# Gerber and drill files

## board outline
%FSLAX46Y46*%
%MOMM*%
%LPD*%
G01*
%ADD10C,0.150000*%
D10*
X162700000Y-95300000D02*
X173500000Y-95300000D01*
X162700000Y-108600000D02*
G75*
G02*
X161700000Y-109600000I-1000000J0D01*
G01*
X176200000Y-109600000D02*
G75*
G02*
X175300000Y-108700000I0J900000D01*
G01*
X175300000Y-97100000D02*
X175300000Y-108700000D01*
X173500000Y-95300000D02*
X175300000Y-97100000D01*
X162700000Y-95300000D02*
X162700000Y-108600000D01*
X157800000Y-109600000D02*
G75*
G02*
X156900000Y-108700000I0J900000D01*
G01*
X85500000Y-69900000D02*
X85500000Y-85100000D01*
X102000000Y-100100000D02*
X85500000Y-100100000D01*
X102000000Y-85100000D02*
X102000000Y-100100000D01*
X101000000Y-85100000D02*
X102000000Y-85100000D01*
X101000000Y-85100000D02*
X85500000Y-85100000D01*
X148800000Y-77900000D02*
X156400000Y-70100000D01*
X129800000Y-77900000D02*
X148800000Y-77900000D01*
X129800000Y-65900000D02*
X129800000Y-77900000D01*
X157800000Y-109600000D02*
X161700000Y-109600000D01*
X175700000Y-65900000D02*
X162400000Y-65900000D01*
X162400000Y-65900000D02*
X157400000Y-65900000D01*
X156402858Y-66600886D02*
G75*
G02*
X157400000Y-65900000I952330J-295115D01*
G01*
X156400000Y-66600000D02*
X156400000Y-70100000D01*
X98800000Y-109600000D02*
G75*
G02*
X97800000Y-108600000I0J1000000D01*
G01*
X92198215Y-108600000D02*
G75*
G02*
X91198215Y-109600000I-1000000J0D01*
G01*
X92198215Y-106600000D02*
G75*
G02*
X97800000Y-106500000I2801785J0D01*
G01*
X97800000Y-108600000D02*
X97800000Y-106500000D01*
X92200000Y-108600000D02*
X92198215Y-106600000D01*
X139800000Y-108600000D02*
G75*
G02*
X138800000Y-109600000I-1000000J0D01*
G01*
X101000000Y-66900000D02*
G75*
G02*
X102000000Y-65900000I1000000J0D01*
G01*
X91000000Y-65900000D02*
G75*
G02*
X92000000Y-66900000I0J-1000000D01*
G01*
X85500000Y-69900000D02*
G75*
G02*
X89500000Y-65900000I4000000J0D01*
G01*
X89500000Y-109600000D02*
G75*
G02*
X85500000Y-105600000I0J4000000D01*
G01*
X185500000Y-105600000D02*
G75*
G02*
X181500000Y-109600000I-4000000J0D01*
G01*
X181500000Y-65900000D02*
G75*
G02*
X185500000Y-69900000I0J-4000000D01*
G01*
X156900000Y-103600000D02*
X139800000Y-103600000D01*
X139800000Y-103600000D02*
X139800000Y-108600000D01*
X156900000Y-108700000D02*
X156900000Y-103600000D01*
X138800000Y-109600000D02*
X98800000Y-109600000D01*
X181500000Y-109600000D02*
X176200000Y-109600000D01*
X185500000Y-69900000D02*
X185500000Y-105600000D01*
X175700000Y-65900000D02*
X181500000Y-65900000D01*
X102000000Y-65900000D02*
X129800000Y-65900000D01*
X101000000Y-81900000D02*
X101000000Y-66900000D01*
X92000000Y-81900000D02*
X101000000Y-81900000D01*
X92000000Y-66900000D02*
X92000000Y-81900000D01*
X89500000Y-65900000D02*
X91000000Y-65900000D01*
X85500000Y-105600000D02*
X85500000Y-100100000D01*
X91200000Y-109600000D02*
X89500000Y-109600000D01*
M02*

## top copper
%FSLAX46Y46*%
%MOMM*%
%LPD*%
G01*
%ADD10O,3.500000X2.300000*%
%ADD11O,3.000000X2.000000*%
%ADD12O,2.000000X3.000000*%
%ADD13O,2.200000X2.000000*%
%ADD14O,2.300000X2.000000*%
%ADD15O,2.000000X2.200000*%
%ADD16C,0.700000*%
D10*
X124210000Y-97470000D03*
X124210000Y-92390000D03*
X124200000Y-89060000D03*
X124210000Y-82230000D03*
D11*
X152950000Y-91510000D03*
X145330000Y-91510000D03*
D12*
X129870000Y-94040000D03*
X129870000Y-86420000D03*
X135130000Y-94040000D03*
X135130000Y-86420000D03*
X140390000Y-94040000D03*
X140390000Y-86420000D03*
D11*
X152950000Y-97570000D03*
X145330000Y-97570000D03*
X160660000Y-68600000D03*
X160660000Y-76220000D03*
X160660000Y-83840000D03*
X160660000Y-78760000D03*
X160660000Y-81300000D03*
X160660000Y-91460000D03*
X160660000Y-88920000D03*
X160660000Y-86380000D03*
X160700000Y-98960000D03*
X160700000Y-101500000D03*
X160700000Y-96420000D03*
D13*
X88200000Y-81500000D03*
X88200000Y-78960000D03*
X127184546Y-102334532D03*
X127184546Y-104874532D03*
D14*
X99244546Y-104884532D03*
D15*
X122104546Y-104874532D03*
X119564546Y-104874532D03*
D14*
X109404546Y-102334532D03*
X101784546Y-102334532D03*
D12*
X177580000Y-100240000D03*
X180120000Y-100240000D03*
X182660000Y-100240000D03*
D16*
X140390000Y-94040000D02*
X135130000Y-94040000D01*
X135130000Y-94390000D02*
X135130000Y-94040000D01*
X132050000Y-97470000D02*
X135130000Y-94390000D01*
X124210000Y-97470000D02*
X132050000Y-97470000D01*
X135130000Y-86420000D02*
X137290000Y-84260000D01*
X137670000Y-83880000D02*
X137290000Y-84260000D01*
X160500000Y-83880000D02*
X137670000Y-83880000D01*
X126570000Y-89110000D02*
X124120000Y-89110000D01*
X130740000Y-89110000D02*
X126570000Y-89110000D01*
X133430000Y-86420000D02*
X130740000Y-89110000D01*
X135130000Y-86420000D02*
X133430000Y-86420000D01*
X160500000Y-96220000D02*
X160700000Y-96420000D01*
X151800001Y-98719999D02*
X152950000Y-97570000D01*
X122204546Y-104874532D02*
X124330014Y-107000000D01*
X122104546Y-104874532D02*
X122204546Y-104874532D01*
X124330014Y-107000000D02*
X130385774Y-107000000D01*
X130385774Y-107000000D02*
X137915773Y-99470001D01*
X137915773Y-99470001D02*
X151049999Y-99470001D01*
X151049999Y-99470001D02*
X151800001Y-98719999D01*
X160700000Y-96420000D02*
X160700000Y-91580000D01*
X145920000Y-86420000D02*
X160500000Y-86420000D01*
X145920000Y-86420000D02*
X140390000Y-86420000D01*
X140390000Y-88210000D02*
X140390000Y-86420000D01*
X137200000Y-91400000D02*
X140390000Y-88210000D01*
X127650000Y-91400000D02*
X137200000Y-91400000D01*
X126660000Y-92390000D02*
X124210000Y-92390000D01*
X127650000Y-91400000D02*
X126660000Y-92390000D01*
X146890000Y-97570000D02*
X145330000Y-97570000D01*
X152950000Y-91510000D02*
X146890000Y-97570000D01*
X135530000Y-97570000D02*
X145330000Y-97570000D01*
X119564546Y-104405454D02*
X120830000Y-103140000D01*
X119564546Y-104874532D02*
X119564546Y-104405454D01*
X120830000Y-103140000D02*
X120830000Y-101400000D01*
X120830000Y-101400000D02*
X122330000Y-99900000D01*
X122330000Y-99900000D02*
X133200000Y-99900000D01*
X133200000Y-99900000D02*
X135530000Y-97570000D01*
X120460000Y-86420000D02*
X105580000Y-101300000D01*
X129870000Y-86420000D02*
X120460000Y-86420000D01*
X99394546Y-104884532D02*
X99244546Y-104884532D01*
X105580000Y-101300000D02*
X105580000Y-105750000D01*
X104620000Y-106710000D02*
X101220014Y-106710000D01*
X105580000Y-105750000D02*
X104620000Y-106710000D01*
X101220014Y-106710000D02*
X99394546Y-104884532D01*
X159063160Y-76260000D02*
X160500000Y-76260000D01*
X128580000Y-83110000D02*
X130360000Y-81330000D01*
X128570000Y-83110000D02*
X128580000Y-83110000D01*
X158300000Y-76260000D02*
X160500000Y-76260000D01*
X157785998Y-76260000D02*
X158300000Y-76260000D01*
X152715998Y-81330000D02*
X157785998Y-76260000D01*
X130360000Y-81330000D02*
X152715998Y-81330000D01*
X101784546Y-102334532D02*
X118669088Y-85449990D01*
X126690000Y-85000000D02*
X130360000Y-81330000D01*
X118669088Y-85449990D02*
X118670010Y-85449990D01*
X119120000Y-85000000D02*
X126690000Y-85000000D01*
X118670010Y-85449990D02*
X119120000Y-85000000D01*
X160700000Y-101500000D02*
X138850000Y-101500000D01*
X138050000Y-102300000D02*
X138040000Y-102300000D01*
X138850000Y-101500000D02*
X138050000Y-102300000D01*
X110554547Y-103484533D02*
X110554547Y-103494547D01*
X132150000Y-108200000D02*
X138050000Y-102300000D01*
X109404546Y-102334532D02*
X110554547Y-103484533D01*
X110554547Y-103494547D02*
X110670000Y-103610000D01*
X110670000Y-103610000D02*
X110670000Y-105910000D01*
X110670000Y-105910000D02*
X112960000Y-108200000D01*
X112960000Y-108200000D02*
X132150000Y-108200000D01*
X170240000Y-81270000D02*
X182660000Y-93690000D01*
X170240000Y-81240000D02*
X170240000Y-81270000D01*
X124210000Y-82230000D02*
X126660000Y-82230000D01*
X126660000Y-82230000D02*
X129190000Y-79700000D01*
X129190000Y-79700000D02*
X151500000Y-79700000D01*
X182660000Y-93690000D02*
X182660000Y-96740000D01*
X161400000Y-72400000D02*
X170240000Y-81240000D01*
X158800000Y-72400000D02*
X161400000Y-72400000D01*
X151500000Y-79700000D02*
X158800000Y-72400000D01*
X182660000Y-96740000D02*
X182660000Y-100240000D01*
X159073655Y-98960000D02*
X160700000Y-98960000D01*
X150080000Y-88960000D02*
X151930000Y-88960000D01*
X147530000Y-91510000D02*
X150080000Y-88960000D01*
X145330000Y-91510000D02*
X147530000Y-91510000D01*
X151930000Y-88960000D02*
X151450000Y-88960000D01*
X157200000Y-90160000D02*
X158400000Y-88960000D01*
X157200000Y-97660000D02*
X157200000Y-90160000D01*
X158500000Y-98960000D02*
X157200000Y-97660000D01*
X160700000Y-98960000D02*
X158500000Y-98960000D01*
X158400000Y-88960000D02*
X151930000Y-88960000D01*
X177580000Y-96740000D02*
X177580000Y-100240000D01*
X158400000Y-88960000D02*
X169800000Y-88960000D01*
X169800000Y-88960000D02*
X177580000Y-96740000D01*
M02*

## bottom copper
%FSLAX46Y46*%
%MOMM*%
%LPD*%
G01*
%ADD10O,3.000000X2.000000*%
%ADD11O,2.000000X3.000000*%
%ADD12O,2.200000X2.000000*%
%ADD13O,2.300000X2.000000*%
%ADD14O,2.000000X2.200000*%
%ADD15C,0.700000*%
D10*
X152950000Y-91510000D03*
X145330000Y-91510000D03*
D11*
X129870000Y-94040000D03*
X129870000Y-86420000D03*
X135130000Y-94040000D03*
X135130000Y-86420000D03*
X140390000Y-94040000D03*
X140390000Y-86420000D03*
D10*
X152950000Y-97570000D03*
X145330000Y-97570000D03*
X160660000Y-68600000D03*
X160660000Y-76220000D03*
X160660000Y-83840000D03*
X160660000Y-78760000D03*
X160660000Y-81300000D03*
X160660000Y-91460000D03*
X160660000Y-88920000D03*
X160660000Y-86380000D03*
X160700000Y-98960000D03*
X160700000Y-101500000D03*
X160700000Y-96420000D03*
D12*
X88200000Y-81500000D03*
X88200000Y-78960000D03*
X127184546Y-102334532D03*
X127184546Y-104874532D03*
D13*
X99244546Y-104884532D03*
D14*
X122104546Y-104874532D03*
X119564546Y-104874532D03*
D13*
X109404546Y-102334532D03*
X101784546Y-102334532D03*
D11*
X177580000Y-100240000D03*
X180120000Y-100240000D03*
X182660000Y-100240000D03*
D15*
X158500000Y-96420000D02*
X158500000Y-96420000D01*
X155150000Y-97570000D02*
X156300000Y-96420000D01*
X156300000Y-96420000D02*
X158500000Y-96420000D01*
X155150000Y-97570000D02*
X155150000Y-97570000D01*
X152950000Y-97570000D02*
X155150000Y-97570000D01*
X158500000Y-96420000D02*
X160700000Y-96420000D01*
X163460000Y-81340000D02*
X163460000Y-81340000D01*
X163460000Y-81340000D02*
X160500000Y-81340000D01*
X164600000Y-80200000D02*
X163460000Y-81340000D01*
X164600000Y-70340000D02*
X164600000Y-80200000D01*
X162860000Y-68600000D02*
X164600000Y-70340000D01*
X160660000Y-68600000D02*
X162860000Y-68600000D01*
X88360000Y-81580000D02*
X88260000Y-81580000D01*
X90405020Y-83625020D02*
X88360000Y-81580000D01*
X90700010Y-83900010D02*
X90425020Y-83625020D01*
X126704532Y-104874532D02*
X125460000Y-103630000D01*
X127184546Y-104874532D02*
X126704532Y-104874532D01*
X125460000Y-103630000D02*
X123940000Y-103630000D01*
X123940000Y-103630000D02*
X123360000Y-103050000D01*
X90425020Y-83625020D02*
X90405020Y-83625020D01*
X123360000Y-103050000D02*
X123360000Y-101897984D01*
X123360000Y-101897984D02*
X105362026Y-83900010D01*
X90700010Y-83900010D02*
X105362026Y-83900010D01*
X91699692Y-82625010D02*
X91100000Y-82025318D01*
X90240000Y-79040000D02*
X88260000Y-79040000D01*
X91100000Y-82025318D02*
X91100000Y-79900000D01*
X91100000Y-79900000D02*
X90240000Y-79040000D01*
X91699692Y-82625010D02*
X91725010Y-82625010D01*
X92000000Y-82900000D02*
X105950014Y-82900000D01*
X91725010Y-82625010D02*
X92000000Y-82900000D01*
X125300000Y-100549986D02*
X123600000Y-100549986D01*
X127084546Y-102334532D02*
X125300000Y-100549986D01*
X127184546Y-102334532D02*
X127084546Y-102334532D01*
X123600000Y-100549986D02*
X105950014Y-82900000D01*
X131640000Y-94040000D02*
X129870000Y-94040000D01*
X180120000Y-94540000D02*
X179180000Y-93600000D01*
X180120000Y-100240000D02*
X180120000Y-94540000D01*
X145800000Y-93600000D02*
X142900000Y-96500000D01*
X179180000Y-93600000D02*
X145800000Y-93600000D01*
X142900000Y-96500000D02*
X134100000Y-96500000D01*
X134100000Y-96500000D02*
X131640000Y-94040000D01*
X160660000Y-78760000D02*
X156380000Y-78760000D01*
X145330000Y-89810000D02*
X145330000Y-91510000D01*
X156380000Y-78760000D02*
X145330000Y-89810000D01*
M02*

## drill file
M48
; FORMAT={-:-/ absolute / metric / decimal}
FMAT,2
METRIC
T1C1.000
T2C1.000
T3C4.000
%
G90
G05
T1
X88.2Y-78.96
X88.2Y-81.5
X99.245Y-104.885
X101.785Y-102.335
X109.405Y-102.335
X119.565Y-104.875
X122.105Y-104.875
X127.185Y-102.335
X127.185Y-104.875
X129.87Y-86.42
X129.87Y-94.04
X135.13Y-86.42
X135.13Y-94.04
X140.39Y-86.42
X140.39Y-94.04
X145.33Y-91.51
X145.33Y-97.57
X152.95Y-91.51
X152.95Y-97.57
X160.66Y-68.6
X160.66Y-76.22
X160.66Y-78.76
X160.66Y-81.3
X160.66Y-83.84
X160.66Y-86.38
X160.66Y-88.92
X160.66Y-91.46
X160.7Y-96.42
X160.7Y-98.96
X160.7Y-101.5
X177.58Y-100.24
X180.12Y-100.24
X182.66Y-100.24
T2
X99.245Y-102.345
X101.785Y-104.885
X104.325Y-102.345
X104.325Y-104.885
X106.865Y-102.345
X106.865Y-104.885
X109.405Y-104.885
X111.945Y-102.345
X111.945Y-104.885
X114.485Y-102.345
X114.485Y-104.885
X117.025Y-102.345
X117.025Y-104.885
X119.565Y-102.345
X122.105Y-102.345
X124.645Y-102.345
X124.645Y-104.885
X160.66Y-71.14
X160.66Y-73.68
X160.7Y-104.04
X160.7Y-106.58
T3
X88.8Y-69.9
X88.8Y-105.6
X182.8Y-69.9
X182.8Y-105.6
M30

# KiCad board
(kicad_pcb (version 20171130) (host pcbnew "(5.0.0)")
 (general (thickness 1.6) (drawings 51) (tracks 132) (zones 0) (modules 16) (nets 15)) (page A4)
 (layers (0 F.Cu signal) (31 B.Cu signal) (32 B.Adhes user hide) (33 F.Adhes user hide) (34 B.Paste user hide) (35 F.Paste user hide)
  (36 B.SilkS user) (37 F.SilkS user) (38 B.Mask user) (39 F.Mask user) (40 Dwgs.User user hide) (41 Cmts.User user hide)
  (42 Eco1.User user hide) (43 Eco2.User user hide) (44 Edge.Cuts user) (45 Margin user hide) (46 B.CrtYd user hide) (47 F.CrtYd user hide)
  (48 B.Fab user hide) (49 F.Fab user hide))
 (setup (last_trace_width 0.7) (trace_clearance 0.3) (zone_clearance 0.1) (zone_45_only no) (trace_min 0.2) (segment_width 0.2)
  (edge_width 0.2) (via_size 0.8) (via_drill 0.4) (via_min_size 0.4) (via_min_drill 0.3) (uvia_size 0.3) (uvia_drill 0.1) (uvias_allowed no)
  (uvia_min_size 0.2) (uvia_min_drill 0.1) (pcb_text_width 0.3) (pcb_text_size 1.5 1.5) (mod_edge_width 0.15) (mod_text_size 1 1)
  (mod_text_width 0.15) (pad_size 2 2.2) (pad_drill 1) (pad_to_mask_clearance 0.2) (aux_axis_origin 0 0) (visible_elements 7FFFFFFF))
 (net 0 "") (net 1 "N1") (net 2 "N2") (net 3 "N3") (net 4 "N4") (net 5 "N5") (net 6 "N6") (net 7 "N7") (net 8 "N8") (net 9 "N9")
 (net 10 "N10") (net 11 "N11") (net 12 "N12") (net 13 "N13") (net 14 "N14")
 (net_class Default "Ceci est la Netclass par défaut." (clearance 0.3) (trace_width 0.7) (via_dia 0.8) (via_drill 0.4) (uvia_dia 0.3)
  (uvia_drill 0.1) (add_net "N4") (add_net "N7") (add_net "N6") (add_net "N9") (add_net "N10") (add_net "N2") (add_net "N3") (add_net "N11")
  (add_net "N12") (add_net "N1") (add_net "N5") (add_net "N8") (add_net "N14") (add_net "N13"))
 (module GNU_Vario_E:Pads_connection (layer F.Cu) (at 124.21 84.77)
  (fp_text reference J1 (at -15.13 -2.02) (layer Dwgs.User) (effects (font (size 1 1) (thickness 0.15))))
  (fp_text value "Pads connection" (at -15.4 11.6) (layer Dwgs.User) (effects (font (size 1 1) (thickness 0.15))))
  (pad 5 smd oval (at 0 12.7) (size 3.5 2.3) (layers F.Cu F.Mask) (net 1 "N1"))
  (pad 4 smd oval (at 0 7.62) (size 3.5 2.3) (layers F.Cu F.Mask) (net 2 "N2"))
  (pad 3 smd oval (at -0.01 4.29) (size 3.5 2.3) (layers F.Cu F.Mask) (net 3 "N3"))
  (pad 1 smd oval (at 0 -2.54) (size 3.5 2.3) (layers F.Cu F.Mask) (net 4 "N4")))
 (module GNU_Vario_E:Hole (layer F.Cu) (at 182.8 105.6)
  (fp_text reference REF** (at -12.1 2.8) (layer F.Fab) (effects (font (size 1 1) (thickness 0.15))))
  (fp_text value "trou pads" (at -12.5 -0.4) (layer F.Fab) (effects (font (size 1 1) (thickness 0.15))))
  (pad "" np_thru_hole circle (at 0 0) (size 4 4) (drill 4) (layers *.Cu *.Mask)))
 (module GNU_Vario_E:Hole (layer F.Cu) (at 182.8 69.9)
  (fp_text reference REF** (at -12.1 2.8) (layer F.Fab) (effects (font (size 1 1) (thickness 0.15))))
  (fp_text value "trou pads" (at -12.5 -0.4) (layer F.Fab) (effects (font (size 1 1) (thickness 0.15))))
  (pad "" np_thru_hole circle (at 0 0) (size 4 4) (drill 4) (layers *.Cu *.Mask)))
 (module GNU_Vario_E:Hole (layer F.Cu) (at 88.8 69.9)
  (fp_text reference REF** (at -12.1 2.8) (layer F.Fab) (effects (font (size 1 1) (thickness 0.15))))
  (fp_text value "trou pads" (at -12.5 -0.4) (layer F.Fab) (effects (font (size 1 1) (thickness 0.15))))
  (pad "" np_thru_hole circle (at 0 0) (size 4 4) (drill 4) (layers *.Cu *.Mask)))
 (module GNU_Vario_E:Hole (layer F.Cu) (at 88.8 105.6)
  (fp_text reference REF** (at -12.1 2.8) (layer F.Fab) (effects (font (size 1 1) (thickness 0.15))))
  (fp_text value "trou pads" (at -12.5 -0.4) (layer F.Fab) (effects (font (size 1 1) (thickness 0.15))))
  (pad "" np_thru_hole circle (at 0 0) (size 4 4) (drill 4) (layers *.Cu *.Mask)))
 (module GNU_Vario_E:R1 (layer F.Cu) (at 145.33 91.51 270)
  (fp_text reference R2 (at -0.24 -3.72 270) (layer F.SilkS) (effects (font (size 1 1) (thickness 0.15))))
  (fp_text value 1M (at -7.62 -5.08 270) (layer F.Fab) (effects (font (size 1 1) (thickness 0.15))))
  (pad 2 thru_hole oval (at 0 -7.62 270) (size 2 3) (drill 1) (layers *.Cu *.Mask) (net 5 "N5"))
  (pad 1 thru_hole oval (at 0 0 270) (size 2 3) (drill 1) (layers *.Cu *.Mask) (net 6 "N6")))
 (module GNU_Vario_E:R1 (layer F.Cu) (at 129.87 86.42 180)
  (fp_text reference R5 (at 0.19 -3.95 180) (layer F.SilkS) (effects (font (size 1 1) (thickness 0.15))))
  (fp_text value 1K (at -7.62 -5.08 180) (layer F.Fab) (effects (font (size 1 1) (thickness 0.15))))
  (pad 2 thru_hole oval (at 0 -7.62 180) (size 2 3) (drill 1) (layers *.Cu *.Mask) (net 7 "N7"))
  (pad 1 thru_hole oval (at 0 0 180) (size 2 3) (drill 1) (layers *.Cu *.Mask) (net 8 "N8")))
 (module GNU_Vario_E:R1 (layer F.Cu) (at 135.13 86.42 180)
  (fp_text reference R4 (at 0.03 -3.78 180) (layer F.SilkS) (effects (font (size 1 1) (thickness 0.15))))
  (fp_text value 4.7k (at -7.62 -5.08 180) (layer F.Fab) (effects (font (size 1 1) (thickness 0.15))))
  (pad 2 thru_hole oval (at 0 -7.62 180) (size 2 3) (drill 1) (layers *.Cu *.Mask) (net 1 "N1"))
  (pad 1 thru_hole oval (at 0 0 180) (size 2 3) (drill 1) (layers *.Cu *.Mask) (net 3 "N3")))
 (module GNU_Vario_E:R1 (layer F.Cu) (at 140.39 86.42 180)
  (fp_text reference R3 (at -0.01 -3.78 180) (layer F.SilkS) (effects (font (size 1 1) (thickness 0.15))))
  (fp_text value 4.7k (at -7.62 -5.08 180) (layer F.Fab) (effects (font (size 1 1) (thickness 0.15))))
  (pad 2 thru_hole oval (at 0 -7.62 180) (size 2 3) (drill 1) (layers *.Cu *.Mask) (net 1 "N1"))
  (pad 1 thru_hole oval (at 0 0 180) (size 2 3) (drill 1) (layers *.Cu *.Mask) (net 2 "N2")))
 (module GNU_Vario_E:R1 (layer F.Cu) (at 145.33 97.57 270)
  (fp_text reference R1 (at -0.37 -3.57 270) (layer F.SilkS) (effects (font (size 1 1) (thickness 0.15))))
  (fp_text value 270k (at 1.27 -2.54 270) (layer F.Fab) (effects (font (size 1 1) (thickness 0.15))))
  (pad 2 thru_hole oval (at 0 -7.62 270) (size 2 3) (drill 1) (layers *.Cu *.Mask) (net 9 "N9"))
  (pad 1 thru_hole oval (at 0 0 270) (size 2 3) (drill 1) (layers *.Cu *.Mask) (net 5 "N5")))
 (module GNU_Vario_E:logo (layer F.Cu) (at 118.22 85.87 90)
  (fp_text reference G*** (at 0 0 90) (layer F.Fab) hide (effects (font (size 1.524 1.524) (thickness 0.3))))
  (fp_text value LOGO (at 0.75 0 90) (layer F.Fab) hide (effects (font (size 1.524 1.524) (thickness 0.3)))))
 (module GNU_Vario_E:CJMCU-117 (layer F.Cu) (at 163.2 81.3 90)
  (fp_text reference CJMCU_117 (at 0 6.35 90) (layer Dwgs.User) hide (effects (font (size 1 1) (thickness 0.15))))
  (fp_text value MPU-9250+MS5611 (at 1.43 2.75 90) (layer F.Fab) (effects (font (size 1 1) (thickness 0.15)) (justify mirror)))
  (pad 10 thru_hole oval (at 12.7 -2.54 90) (size 2 3) (drill 1) (layers *.Cu *.Mask) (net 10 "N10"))
  (pad 7 thru_hole oval (at 5.08 -2.54 90) (size 2 3) (drill 1) (layers *.Cu *.Mask) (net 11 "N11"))
  (pad 4 thru_hole oval (at -2.54 -2.54 90) (size 2 3) (drill 1) (layers *.Cu *.Mask) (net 3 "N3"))
  (pad 6 thru_hole oval (at 2.54 -2.54 90) (size 2 3) (drill 1) (layers *.Cu *.Mask) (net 6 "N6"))
  (pad 5 thru_hole oval (at 0 -2.54 90) (size 2 3) (drill 1) (layers *.Cu *.Mask) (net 10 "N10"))
  (pad 1 thru_hole oval (at -10.16 -2.54 90) (size 2 3) (drill 1) (layers *.Cu *.Mask) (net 9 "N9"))
  (pad 2 thru_hole oval (at -7.62 -2.54 90) (size 2 3) (drill 1) (layers *.Cu *.Mask) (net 6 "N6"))
  (pad 3 thru_hole oval (at -5.08 -2.54 90) (size 2 3) (drill 1) (layers *.Cu *.Mask) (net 2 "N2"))
  (pad "" np_thru_hole circle (at 7.62 -2.54 90) (size 1 1) (drill 1) (layers *.Cu *.Mask))
  (pad "" np_thru_hole circle (at 10.16 -2.54 90) (size 1 1) (drill 1) (layers *.Cu *.Mask)))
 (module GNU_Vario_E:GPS (layer F.Cu) (at 160.7 96.42 270)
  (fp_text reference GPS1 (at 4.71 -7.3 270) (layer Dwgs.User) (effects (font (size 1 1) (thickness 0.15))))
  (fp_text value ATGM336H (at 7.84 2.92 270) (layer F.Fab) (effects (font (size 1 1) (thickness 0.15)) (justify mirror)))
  (pad 2 thru_hole oval (at 2.54 0 270) (size 2 3) (drill 1) (layers *.Cu *.Mask) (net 6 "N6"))
  (pad 3 thru_hole oval (at 5.08 0 270) (size 2 3) (drill 1) (layers *.Cu *.Mask) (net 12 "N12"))
  (pad 1 thru_hole oval (at 0 0 270) (size 2 3) (drill 1) (layers *.Cu *.Mask) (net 9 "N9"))
  (pad "" np_thru_hole circle (at 7.62 0 270) (size 1 1) (drill 1) (layers *.Cu *.Mask))
  (pad "" np_thru_hole circle (at 10.16 0 270) (size 1 1) (drill 1) (layers *.Cu *.Mask)))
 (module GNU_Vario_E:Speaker (layer F.Cu) (at 90.74 84.04 90)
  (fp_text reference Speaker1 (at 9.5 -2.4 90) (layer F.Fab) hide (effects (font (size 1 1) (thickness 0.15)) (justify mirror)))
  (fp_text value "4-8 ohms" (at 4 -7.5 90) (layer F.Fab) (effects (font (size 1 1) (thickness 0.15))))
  (pad 2 thru_hole oval (at 2.54 -2.54 90) (size 2 2.2) (drill 1) (layers *.Cu *.Mask) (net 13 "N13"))
  (pad 1 thru_hole oval (at 5.08 -2.54 90) (size 2 2.2) (drill 1) (layers *.Cu *.Mask) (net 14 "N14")))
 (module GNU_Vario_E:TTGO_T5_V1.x (layer F.Cu) (at 127.734546 102.554532 90)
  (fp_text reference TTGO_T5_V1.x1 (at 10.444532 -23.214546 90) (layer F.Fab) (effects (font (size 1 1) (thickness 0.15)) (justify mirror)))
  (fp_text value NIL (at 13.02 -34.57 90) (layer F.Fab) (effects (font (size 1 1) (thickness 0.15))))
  (pad "" np_thru_hole circle (at 0.21 -28.49 90) (size 1 1) (drill 1) (layers *.Cu *.Mask))
  (pad "" np_thru_hole circle (at 0.21 -23.41 90) (size 1 1) (drill 1) (layers *.Cu *.Mask))
  (pad "" np_thru_hole circle (at 0.21 -20.87 90) (size 1 1) (drill 1) (layers *.Cu *.Mask))
  (pad "" np_thru_hole circle (at -2.33 -3.09 90) (size 1 1) (drill 1) (layers *.Cu *.Mask))
  (pad "" np_thru_hole circle (at 0.21 -3.09 90) (size 1 1) (drill 1) (layers *.Cu *.Mask))
  (pad "" np_thru_hole circle (at 0.21 -5.63 90) (size 1 1) (drill 1) (layers *.Cu *.Mask))
  (pad "" np_thru_hole circle (at 0.21 -15.79 90) (size 1 1) (drill 1) (layers *.Cu *.Mask))
  (pad "" np_thru_hole circle (at 0.21 -13.25 90) (size 1 1) (drill 1) (layers *.Cu *.Mask))
  (pad "" np_thru_hole circle (at 0.21 -8.17 90) (size 1 1) (drill 1) (layers *.Cu *.Mask))
  (pad "" np_thru_hole circle (at 0.21 -10.71 90) (size 1 1) (drill 1) (layers *.Cu *.Mask))
  (pad "" np_thru_hole circle (at -2.33 -10.71 90) (size 1 1) (drill 1) (layers *.Cu *.Mask))
  (pad "" np_thru_hole circle (at -2.33 -13.25 90) (size 1 1) (drill 1) (layers *.Cu *.Mask))
  (pad "" np_thru_hole circle (at -2.33 -15.79 90) (size 1 1) (drill 1) (layers *.Cu *.Mask))
  (pad "" np_thru_hole circle (at -2.33 -18.33 90) (size 1 1) (drill 1) (layers *.Cu *.Mask))
  (pad "" np_thru_hole circle (at -2.33 -20.87 90) (size 1 1) (drill 1) (layers *.Cu *.Mask))
  (pad "" np_thru_hole circle (at -2.33 -23.41 90) (size 1 1) (drill 1) (layers *.Cu *.Mask))
  (pad "" np_thru_hole circle (at -2.33 -25.95 90) (size 1 1) (drill 1) (layers *.Cu *.Mask))
  (pad 13 thru_hole oval (at 0.22 -0.55 90) (size 2 2.2) (drill 1) (layers *.Cu *.Mask) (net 14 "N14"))
  (pad 1 thru_hole oval (at -2.32 -0.55 90) (size 2 2.2) (drill 1) (layers *.Cu *.Mask) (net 13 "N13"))
  (pad 12 thru_hole oval (at -2.33 -28.49 90) (size 2 2.3) (drill 1) (layers *.Cu *.Mask) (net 8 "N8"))
  (pad 3 thru_hole oval (at -2.32 -5.63 90) (size 2.2 2) (drill 1) (layers *.Cu *.Mask) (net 9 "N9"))
  (pad 4 thru_hole oval (at -2.32 -8.17 90) (size 2.2 2) (drill 1) (layers *.Cu *.Mask) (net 5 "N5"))
  (pad 20 thru_hole oval (at 0.22 -18.33 90) (size 2 2.3) (drill 1) (layers *.Cu *.Mask) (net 12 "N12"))
  (pad 23 thru_hole oval (at 0.22 -25.95 90) (size 2 2.3) (drill 1) (layers *.Cu *.Mask) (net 11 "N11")))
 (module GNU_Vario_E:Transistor (layer F.Cu) (at 185.2 97.7 180)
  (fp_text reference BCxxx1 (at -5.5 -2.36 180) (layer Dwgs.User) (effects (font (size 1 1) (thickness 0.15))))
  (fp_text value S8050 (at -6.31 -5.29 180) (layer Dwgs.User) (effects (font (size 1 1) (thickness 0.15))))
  (pad 3 thru_hole oval (at 7.62 -2.54 180) (size 2 3) (drill 1) (layers *.Cu *.Mask) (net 6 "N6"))
  (pad 2 thru_hole oval (at 5.08 -2.54 180) (size 2 3) (drill 1) (layers *.Cu *.Mask) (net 7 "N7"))
  (pad 1 thru_hole oval (at 2.54 -2.54 180) (size 2 3) (drill 1) (layers *.Cu *.Mask) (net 4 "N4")))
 (gr_line (start 162.7 95.3) (end 173.5 95.3) (layer Edge.Cuts) (width 0.15))
 (gr_arc (start 161.7 108.6) (end 161.7 109.6) (angle -90) (layer Edge.Cuts) (width 0.15))
 (gr_arc (start 176.2 108.7) (end 175.3 108.7) (angle -90) (layer Edge.Cuts) (width 0.15))
 (gr_line (start 175.3 97.1) (end 175.3 108.7) (layer Edge.Cuts) (width 0.15))
 (gr_line (start 173.5 95.3) (end 175.3 97.1) (layer Edge.Cuts) (width 0.15))
 (gr_line (start 162.7 95.3) (end 162.7 108.6) (layer Edge.Cuts) (width 0.15))
 (gr_arc (start 157.8 108.7) (end 156.9 108.7) (angle -90) (layer Edge.Cuts) (width 0.15))
 (gr_line (start 85.5 69.9) (end 85.5 85.1) (layer Edge.Cuts) (width 0.15))
 (gr_line (start 102 100.1) (end 85.5 100.1) (layer Edge.Cuts) (width 0.15))
 (gr_line (start 102 85.1) (end 102 100.1) (layer Edge.Cuts) (width 0.15))
 (gr_line (start 101 85.1) (end 102 85.1) (layer Edge.Cuts) (width 0.15))
 (gr_line (start 101 85.1) (end 85.5 85.1) (layer Edge.Cuts) (width 0.15))
 (gr_line (start 148.8 77.9) (end 156.4 70.1) (layer Edge.Cuts) (width 0.15))
 (gr_line (start 129.8 77.9) (end 148.8 77.9) (layer Edge.Cuts) (width 0.15))
 (gr_line (start 129.8 65.9) (end 129.8 77.9) (layer Edge.Cuts) (width 0.15))
 (gr_line (start 157.8 109.6) (end 161.7 109.6) (layer Edge.Cuts) (width 0.15))
 (gr_line (start 175.7 65.9) (end 162.4 65.9) (layer Edge.Cuts) (width 0.15))
 (gr_line (start 162.4 65.9) (end 157.4 65.9) (layer Edge.Cuts) (width 0.15))
 (gr_arc (start 157.355188 66.896001) (end 157.4 65.9) (angle -75.35856355) (layer Edge.Cuts) (width 0.15))
 (gr_line (start 156.4 66.6) (end 156.4 70.1) (layer Edge.Cuts) (width 0.15))
 (gr_arc (start 98.8 108.6) (end 97.8 108.6) (angle -90) (layer Edge.Cuts) (width 0.15))
 (gr_arc (start 91.198215 108.6) (end 91.198215 109.6) (angle -90) (layer Edge.Cuts) (width 0.15))
 (gr_arc (start 95 106.6) (end 97.8 106.5) (angle -177.9545915) (layer Edge.Cuts) (width 0.15))
 (gr_line (start 97.8 108.6) (end 97.8 106.5) (layer Edge.Cuts) (width 0.15))
 (gr_line (start 92.2 108.6) (end 92.198215 106.6) (layer Edge.Cuts) (width 0.15))
 (gr_arc (start 138.8 108.6) (end 138.8 109.6) (angle -90) (layer Edge.Cuts) (width 0.15))
 (gr_arc (start 102 66.9) (end 102 65.9) (angle -90) (layer Edge.Cuts) (width 0.15))
 (gr_arc (start 91 66.9) (end 92 66.9) (angle -90) (layer Edge.Cuts) (width 0.15))
 (gr_arc (start 89.5 69.9) (end 89.5 65.9) (angle -90) (layer Edge.Cuts) (width 0.15))
 (gr_arc (start 89.5 105.6) (end 85.5 105.6) (angle -90) (layer Edge.Cuts) (width 0.15))
 (gr_arc (start 181.5 105.6) (end 181.5 109.6) (angle -90) (layer Edge.Cuts) (width 0.15))
 (gr_arc (start 181.5 69.9) (end 185.5 69.9) (angle -90) (layer Edge.Cuts) (width 0.15))
 (gr_line (start 156.9 103.6) (end 139.8 103.6) (layer Edge.Cuts) (width 0.15))
 (gr_line (start 139.8 103.6) (end 139.8 108.6) (layer Edge.Cuts) (width 0.15))
 (gr_line (start 156.9 108.7) (end 156.9 103.6) (layer Edge.Cuts) (width 0.15))
 (gr_line (start 138.8 109.6) (end 98.8 109.6) (layer Edge.Cuts) (width 0.15))
 (gr_line (start 181.5 109.6) (end 176.2 109.6) (layer Edge.Cuts) (width 0.15))
 (gr_line (start 185.5 69.9) (end 185.5 105.6) (layer Edge.Cuts) (width 0.15))
 (gr_line (start 175.7 65.9) (end 181.5 65.9) (layer Edge.Cuts) (width 0.15))
 (gr_line (start 102 65.9) (end 129.8 65.9) (layer Edge.Cuts) (width 0.15))
 (gr_line (start 101 81.9) (end 101 66.9) (layer Edge.Cuts) (width 0.15))
 (gr_line (start 92 81.9) (end 101 81.9) (layer Edge.Cuts) (width 0.15))
 (gr_line (start 92 66.9) (end 92 81.9) (layer Edge.Cuts) (width 0.15))
 (gr_line (start 89.5 65.9) (end 91 65.9) (layer Edge.Cuts) (width 0.15))
 (gr_line (start 85.5 105.6) (end 85.5 100.1) (layer Edge.Cuts) (width 0.15))
 (gr_line (start 91.2 109.6) (end 89.5 109.6) (layer Edge.Cuts) (width 0.15))
 (segment (start 140.39 94.04) (end 135.13 94.04) (width 0.7) (layer F.Cu) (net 1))
 (segment (start 135.13 94.39) (end 135.13 94.04) (width 0.7) (layer F.Cu) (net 1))
 (segment (start 132.05 97.47) (end 135.13 94.39) (width 0.7) (layer F.Cu) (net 1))
 (segment (start 124.21 97.47) (end 132.05 97.47) (width 0.7) (layer F.Cu) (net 1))
 (segment (start 135.13 86.42) (end 137.29 84.26) (width 0.7) (layer F.Cu) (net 3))
 (segment (start 137.67 83.88) (end 137.29 84.26) (width 0.7) (layer F.Cu) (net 3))
 (segment (start 160.5 83.88) (end 137.67 83.88) (width 0.7) (layer F.Cu) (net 3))
 (segment (start 126.57 89.11) (end 124.12 89.11) (width 0.7) (layer F.Cu) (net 3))
 (segment (start 130.74 89.11) (end 126.57 89.11) (width 0.7) (layer F.Cu) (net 3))
 (segment (start 133.43 86.42) (end 130.74 89.11) (width 0.7) (layer F.Cu) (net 3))
 (segment (start 135.13 86.42) (end 133.43 86.42) (width 0.7) (layer F.Cu) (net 3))
 (segment (start 160.5 96.22) (end 160.7 96.42) (width 0.7) (layer F.Cu) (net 9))
 (segment (start 158.5 96.42) (end 158.5 96.42) (width 0.7) (layer B.Cu) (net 9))
 (segment (start 155.15 97.57) (end 156.3 96.42) (width 0.7) (layer B.Cu) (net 9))
 (segment (start 156.3 96.42) (end 158.5 96.42) (width 0.7) (layer B.Cu) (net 9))
 (segment (start 155.15 97.57) (end 155.15 97.57) (width 0.7) (layer B.Cu) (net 9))
 (segment (start 152.95 97.57) (end 155.15 97.57) (width 0.7) (layer B.Cu) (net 9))
 (segment (start 158.5 96.42) (end 160.7 96.42) (width 0.7) (layer B.Cu) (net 9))
 (segment (start 151.800001 98.719999) (end 152.95 97.57) (width 0.7) (layer F.Cu) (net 9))
 (segment (start 122.204546 104.874532) (end 124.330014 107) (width 0.7) (layer F.Cu) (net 9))
 (segment (start 122.104546 104.874532) (end 122.204546 104.874532) (width 0.7) (layer F.Cu) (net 9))
 (segment (start 124.330014 107) (end 130.385774 107) (width 0.7) (layer F.Cu) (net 9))
 (segment (start 130.385774 107) (end 137.915773 99.470001) (width 0.7) (layer F.Cu) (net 9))
 (segment (start 137.915773 99.470001) (end 151.049999 99.470001) (width 0.7) (layer F.Cu) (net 9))
 (segment (start 151.049999 99.470001) (end 151.800001 98.719999) (width 0.7) (layer F.Cu) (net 9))
 (segment (start 160.7 96.42) (end 160.7 91.58) (width 0.7) (layer F.Cu) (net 9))
 (segment (start 145.92 86.42) (end 160.5 86.42) (width 0.7) (layer F.Cu) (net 2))
 (segment (start 145.92 86.42) (end 140.39 86.42) (width 0.7) (layer F.Cu) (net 2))
 (segment (start 140.39 88.21) (end 140.39 86.42) (width 0.7) (layer F.Cu) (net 2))
 (segment (start 137.2 91.4) (end 140.39 88.21) (width 0.7) (layer F.Cu) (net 2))
 (segment (start 127.65 91.4) (end 137.2 91.4) (width 0.7) (layer F.Cu) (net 2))
 (segment (start 126.66 92.39) (end 124.21 92.39) (width 0.7) (layer F.Cu) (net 2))
 (segment (start 127.65 91.4) (end 126.66 92.39) (width 0.7) (layer F.Cu) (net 2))
 (segment (start 146.89 97.57) (end 145.33 97.57) (width 0.7) (layer F.Cu) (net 5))
 (segment (start 152.95 91.51) (end 146.89 97.57) (width 0.7) (layer F.Cu) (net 5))
 (segment (start 135.53 97.57) (end 145.33 97.57) (width 0.7) (layer F.Cu) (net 5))
 (segment (start 119.564546 104.405454) (end 120.83 103.14) (width 0.7) (layer F.Cu) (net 5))
 (segment (start 119.564546 104.874532) (end 119.564546 104.405454) (width 0.7) (layer F.Cu) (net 5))
 (segment (start 120.83 103.14) (end 120.83 101.4) (width 0.7) (layer F.Cu) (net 5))
 (segment (start 120.83 101.4) (end 122.33 99.9) (width 0.7) (layer F.Cu) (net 5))
 (segment (start 122.33 99.9) (end 133.2 99.9) (width 0.7) (layer F.Cu) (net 5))
 (segment (start 133.2 99.9) (end 135.53 97.57) (width 0.7) (layer F.Cu) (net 5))
 (segment (start 120.46 86.42) (end 105.58 101.3) (width 0.7) (layer F.Cu) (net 8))
 (segment (start 129.87 86.42) (end 120.46 86.42) (width 0.7) (layer F.Cu) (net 8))
 (segment (start 99.394546 104.884532) (end 99.244546 104.884532) (width 0.7) (layer F.Cu) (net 8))
 (segment (start 105.58 101.3) (end 105.58 105.75) (width 0.7) (layer F.Cu) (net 8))
 (segment (start 104.62 106.71) (end 101.220014 106.71) (width 0.7) (layer F.Cu) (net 8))
 (segment (start 105.58 105.75) (end 104.62 106.71) (width 0.7) (layer F.Cu) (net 8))
 (segment (start 101.220014 106.71) (end 99.394546 104.884532) (width 0.7) (layer F.Cu) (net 8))
 (segment (start 163.46 81.34) (end 163.46 81.34) (width 0.7) (layer B.Cu) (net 10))
 (segment (start 163.46 81.34) (end 160.5 81.34) (width 0.7) (layer B.Cu) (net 10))
 (segment (start 164.6 80.2) (end 163.46 81.34) (width 0.7) (layer B.Cu) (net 10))
 (segment (start 164.6 70.34) (end 164.6 80.2) (width 0.7) (layer B.Cu) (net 10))
 (segment (start 162.86 68.6) (end 164.6 70.34) (width 0.7) (layer B.Cu) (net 10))
 (segment (start 160.66 68.6) (end 162.86 68.6) (width 0.7) (layer B.Cu) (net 10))
 (segment (start 159.06316 76.26) (end 160.5 76.26) (width 0.7) (layer F.Cu) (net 11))
 (segment (start 128.58 83.11) (end 130.36 81.33) (width 0.7) (layer F.Cu) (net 11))
 (segment (start 128.57 83.11) (end 128.58 83.11) (width 0.7) (layer F.Cu) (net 11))
 (segment (start 158.3 76.26) (end 160.5 76.26) (width 0.7) (layer F.Cu) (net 11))
 (segment (start 157.785998 76.26) (end 158.3 76.26) (width 0.7) (layer F.Cu) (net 11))
 (segment (start 152.715998 81.33) (end 157.785998 76.26) (width 0.7) (layer F.Cu) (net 11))
 (segment (start 130.36 81.33) (end 152.715998 81.33) (width 0.7) (layer F.Cu) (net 11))
 (segment (start 101.784546 102.334532) (end 118.669088 85.44999) (width 0.7) (layer F.Cu) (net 11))
 (segment (start 126.69 85) (end 130.36 81.33) (width 0.7) (layer F.Cu) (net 11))
 (segment (start 118.669088 85.44999) (end 118.67001 85.44999) (width 0.7) (layer F.Cu) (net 11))
 (segment (start 119.12 85) (end 126.69 85) (width 0.7) (layer F.Cu) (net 11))
 (segment (start 118.67001 85.44999) (end 119.12 85) (width 0.7) (layer F.Cu) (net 11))
 (segment (start 160.7 101.5) (end 138.85 101.5) (width 0.7) (layer F.Cu) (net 12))
 (segment (start 138.05 102.3) (end 138.04 102.3) (width 0.7) (layer F.Cu) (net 12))
 (segment (start 138.85 101.5) (end 138.05 102.3) (width 0.7) (layer F.Cu) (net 12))
 (segment (start 110.554547 103.484533) (end 110.554547 103.494547) (width 0.7) (layer F.Cu) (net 12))
 (segment (start 132.15 108.2) (end 138.05 102.3) (width 0.7) (layer F.Cu) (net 12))
 (segment (start 109.404546 102.334532) (end 110.554547 103.484533) (width 0.7) (layer F.Cu) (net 12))
 (segment (start 110.554547 103.494547) (end 110.67 103.61) (width 0.7) (layer F.Cu) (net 12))
 (segment (start 110.67 103.61) (end 110.67 105.91) (width 0.7) (layer F.Cu) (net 12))
 (segment (start 110.67 105.91) (end 112.96 108.2) (width 0.7) (layer F.Cu) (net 12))
 (segment (start 112.96 108.2) (end 132.15 108.2) (width 0.7) (layer F.Cu) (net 12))
 (segment (start 88.36 81.58) (end 88.26 81.58) (width 0.7) (layer B.Cu) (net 13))
 (segment (start 90.40502 83.62502) (end 88.36 81.58) (width 0.7) (layer B.Cu) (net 13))
 (segment (start 90.70001 83.90001) (end 90.42502 83.62502) (width 0.7) (layer B.Cu) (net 13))
 (segment (start 126.704532 104.874532) (end 125.46 103.63) (width 0.7) (layer B.Cu) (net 13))
 (segment (start 127.184546 104.874532) (end 126.704532 104.874532) (width 0.7) (layer B.Cu) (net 13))
 (segment (start 125.46 103.63) (end 123.94 103.63) (width 0.7) (layer B.Cu) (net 13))
 (segment (start 123.94 103.63) (end 123.36 103.05) (width 0.7) (layer B.Cu) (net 13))
 (segment (start 90.42502 83.62502) (end 90.40502 83.62502) (width 0.7) (layer B.Cu) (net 13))
 (segment (start 123.36 103.05) (end 123.36 101.897984) (width 0.7) (layer B.Cu) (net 13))
 (segment (start 123.36 101.897984) (end 105.362026 83.90001) (width 0.7) (layer B.Cu) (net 13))
 (segment (start 90.70001 83.90001) (end 105.362026 83.90001) (width 0.7) (layer B.Cu) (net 13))
 (segment (start 91.699692 82.62501) (end 91.1 82.025318) (width 0.7) (layer B.Cu) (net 14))
 (segment (start 90.24 79.04) (end 88.26 79.04) (width 0.7) (layer B.Cu) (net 14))
 (segment (start 91.1 82.025318) (end 91.1 79.9) (width 0.7) (layer B.Cu) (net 14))
 (segment (start 91.1 79.9) (end 90.24 79.04) (width 0.7) (layer B.Cu) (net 14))
 (segment (start 91.699692 82.62501) (end 91.72501 82.62501) (width 0.7) (layer B.Cu) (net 14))
 (segment (start 92 82.9) (end 105.950014 82.9) (width 0.7) (layer B.Cu) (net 14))
 (segment (start 91.72501 82.62501) (end 92 82.9) (width 0.7) (layer B.Cu) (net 14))
 (segment (start 125.3 100.549986) (end 123.6 100.549986) (width 0.7) (layer B.Cu) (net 14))
 (segment (start 127.084546 102.334532) (end 125.3 100.549986) (width 0.7) (layer B.Cu) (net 14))
 (segment (start 127.184546 102.334532) (end 127.084546 102.334532) (width 0.7) (layer B.Cu) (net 14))
 (segment (start 123.6 100.549986) (end 105.950014 82.9) (width 0.7) (layer B.Cu) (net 14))
 (segment (start 170.24 81.27) (end 182.66 93.69) (width 0.7) (layer F.Cu) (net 4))
 (segment (start 170.24 81.24) (end 170.24 81.27) (width 0.7) (layer F.Cu) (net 4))
 (segment (start 124.21 82.23) (end 126.66 82.23) (width 0.7) (layer F.Cu) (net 4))
 (segment (start 126.66 82.23) (end 129.19 79.7) (width 0.7) (layer F.Cu) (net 4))
 (segment (start 129.19 79.7) (end 151.5 79.7) (width 0.7) (layer F.Cu) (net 4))
 (segment (start 182.66 93.69) (end 182.66 96.74) (width 0.7) (layer F.Cu) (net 4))
 (segment (start 161.4 72.4) (end 170.24 81.24) (width 0.7) (layer F.Cu) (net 4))
 (segment (start 158.8 72.4) (end 161.4 72.4) (width 0.7) (layer F.Cu) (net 4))
 (segment (start 151.5 79.7) (end 158.8 72.4) (width 0.7) (layer F.Cu) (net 4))
 (segment (start 182.66 96.74) (end 182.66 100.24) (width 0.7) (layer F.Cu) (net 4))
 (segment (start 131.64 94.04) (end 129.87 94.04) (width 0.7) (layer B.Cu) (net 7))
 (segment (start 180.12 94.54) (end 179.18 93.6) (width 0.7) (layer B.Cu) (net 7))
 (segment (start 180.12 100.24) (end 180.12 94.54) (width 0.7) (layer B.Cu) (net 7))
 (segment (start 145.8 93.6) (end 142.9 96.5) (width 0.7) (layer B.Cu) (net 7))
 (segment (start 179.18 93.6) (end 145.8 93.6) (width 0.7) (layer B.Cu) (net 7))
 (segment (start 142.9 96.5) (end 134.1 96.5) (width 0.7) (layer B.Cu) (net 7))
 (segment (start 134.1 96.5) (end 131.64 94.04) (width 0.7) (layer B.Cu) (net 7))
 (segment (start 159.073655 98.96) (end 160.7 98.96) (width 0.7) (layer F.Cu) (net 6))
 (segment (start 150.08 88.96) (end 151.93 88.96) (width 0.7) (layer F.Cu) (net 6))
 (segment (start 147.53 91.51) (end 150.08 88.96) (width 0.7) (layer F.Cu) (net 6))
 (segment (start 145.33 91.51) (end 147.53 91.51) (width 0.7) (layer F.Cu) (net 6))
 (segment (start 151.93 88.96) (end 151.45 88.96) (width 0.7) (layer F.Cu) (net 6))
 (segment (start 157.2 90.16) (end 158.4 88.96) (width 0.7) (layer F.Cu) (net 6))
 (segment (start 157.2 97.66) (end 157.2 90.16) (width 0.7) (layer F.Cu) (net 6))
 (segment (start 158.5 98.96) (end 157.2 97.66) (width 0.7) (layer F.Cu) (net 6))
 (segment (start 160.7 98.96) (end 158.5 98.96) (width 0.7) (layer F.Cu) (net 6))
 (segment (start 158.4 88.96) (end 151.93 88.96) (width 0.7) (layer F.Cu) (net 6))
 (segment (start 177.58 96.74) (end 177.58 100.24) (width 0.7) (layer F.Cu) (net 6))
 (segment (start 158.4 88.96) (end 169.8 88.96) (width 0.7) (layer F.Cu) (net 6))
 (segment (start 169.8 88.96) (end 177.58 96.74) (width 0.7) (layer F.Cu) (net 6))
 (segment (start 160.66 78.76) (end 156.38 78.76) (width 0.7) (layer B.Cu) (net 6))
 (segment (start 145.33 89.81) (end 145.33 91.51) (width 0.7) (layer B.Cu) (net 6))
 (segment (start 156.38 78.76) (end 145.33 89.81) (width 0.7) (layer B.Cu) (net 6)))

